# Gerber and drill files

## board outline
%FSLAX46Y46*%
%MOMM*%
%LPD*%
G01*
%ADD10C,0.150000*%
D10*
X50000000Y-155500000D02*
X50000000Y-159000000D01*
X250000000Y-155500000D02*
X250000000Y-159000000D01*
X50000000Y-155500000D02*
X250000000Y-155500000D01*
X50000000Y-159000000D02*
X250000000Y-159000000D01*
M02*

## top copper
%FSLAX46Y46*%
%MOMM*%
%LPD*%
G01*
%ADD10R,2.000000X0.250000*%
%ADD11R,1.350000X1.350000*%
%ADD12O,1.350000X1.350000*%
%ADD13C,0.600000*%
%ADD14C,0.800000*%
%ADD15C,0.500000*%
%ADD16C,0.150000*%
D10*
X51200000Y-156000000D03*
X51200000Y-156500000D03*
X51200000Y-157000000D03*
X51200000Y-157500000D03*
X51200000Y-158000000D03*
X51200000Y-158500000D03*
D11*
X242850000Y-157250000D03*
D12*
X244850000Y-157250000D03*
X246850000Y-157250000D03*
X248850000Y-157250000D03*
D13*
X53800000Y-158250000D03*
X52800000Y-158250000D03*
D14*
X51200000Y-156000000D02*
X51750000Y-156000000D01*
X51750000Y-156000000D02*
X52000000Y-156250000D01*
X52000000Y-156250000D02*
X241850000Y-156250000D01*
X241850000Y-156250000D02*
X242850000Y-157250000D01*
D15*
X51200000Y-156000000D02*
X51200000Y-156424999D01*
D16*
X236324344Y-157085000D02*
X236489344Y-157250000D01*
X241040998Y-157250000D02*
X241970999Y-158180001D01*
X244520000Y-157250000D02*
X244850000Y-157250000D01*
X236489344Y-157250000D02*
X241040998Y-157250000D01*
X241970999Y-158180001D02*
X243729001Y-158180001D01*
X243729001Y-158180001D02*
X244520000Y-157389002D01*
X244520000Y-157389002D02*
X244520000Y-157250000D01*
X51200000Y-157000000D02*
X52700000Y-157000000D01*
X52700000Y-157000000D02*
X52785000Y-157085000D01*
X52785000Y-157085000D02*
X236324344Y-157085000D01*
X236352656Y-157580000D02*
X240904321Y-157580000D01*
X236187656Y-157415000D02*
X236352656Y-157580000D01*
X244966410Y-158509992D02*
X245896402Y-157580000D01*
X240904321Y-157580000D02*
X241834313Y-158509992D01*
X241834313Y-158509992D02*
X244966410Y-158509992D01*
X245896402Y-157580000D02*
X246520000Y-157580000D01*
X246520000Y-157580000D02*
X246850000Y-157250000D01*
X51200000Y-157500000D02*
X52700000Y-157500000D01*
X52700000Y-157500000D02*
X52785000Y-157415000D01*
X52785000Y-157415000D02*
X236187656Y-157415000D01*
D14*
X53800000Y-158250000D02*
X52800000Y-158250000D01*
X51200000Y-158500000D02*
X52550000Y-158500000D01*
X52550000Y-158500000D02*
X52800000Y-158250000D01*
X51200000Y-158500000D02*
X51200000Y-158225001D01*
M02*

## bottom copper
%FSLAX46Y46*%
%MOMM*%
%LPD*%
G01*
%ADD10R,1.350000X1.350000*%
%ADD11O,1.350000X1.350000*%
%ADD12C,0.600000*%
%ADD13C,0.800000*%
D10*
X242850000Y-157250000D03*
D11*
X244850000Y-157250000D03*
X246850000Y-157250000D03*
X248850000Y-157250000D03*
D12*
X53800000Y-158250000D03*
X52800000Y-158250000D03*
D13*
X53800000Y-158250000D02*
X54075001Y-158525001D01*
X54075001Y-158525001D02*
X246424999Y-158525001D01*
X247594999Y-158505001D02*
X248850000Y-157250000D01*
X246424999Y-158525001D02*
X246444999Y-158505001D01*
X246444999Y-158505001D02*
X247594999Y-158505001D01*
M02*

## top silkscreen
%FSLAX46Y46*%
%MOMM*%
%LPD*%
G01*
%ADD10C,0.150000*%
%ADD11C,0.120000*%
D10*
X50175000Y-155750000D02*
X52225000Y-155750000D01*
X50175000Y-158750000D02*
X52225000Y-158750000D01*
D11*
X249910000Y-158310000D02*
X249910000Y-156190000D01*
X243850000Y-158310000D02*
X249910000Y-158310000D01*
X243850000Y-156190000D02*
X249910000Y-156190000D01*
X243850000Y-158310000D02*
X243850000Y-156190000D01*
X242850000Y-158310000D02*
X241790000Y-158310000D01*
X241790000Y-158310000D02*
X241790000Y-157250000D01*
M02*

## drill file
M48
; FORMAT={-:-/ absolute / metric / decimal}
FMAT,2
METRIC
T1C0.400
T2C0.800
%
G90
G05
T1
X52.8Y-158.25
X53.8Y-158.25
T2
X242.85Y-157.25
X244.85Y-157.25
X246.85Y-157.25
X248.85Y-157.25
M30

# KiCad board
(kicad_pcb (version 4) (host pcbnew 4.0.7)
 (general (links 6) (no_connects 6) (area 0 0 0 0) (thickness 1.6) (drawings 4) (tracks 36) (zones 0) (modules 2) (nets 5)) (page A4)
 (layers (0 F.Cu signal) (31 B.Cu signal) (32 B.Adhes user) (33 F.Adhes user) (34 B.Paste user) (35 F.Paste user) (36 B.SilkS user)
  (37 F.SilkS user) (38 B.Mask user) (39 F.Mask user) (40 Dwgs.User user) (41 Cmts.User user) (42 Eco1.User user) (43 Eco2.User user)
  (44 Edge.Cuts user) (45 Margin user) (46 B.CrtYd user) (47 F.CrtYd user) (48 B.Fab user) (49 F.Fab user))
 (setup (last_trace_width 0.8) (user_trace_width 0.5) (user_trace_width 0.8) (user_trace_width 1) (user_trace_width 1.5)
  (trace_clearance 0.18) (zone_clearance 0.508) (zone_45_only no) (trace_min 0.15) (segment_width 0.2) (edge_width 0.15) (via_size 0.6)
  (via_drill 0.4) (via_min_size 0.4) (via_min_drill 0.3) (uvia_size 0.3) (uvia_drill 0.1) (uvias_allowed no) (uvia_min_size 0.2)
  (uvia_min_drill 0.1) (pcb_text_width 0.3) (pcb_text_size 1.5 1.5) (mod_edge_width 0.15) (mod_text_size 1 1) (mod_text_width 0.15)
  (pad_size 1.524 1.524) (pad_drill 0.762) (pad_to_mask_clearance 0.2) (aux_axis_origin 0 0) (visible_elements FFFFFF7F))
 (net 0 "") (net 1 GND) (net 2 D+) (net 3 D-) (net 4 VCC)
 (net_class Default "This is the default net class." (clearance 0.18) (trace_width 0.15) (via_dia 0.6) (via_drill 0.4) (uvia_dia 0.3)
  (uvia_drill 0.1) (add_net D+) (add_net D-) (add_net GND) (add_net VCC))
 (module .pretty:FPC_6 (layer F.Cu) (at 51.2 157.25 270)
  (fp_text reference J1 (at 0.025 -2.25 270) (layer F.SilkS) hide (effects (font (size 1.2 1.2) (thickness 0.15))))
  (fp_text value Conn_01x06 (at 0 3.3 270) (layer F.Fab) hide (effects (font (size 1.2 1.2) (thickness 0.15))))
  (fp_line (start -1.5 1.025) (end -1.5 -1.025) (layer F.SilkS) (width 0.15))
  (fp_line (start 1.5 1.025) (end 1.5 -1.025) (layer F.SilkS) (width 0.15))
  (pad 1 smd rect (at -1.25 0 270) (size 0.25 2) (layers F.Cu F.Paste F.Mask) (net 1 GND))
  (pad 2 smd rect (at -0.75 0 270) (size 0.25 2) (layers F.Cu F.Paste F.Mask) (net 1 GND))
  (pad 3 smd rect (at -0.25 0 270) (size 0.25 2) (layers F.Cu F.Paste F.Mask) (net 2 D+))
  (pad 4 smd rect (at 0.25 0 270) (size 0.25 2) (layers F.Cu F.Paste F.Mask) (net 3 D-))
  (pad 5 smd rect (at 0.75 0 270) (size 0.25 2) (layers F.Cu F.Paste F.Mask) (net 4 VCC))
  (pad 6 smd rect (at 1.25 0 270) (size 0.25 2) (layers F.Cu F.Paste F.Mask) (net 4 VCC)))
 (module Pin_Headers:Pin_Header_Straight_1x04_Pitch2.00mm (layer F.Cu) (at 242.85 157.25 90)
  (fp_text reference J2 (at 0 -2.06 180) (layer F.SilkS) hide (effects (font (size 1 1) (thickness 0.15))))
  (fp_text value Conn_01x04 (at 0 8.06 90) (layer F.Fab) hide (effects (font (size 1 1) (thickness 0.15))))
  (fp_line (start -1.06 7.06) (end 1.06 7.06) (layer F.SilkS) (width 0.12))
  (fp_line (start -1.06 1) (end -1.06 7.06) (layer F.SilkS) (width 0.12))
  (fp_line (start 1.06 1) (end 1.06 7.06) (layer F.SilkS) (width 0.12))
  (fp_line (start -1.06 1) (end 1.06 1) (layer F.SilkS) (width 0.12))
  (fp_line (start -1.06 0) (end -1.06 -1.06) (layer F.SilkS) (width 0.12))
  (fp_line (start -1.06 -1.06) (end 0 -1.06) (layer F.SilkS) (width 0.12))
  (pad 1 thru_hole rect (at 0 0 90) (size 1.35 1.35) (drill 0.8) (layers *.Cu *.Mask) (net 1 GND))
  (pad 2 thru_hole oval (at 0 2 90) (size 1.35 1.35) (drill 0.8) (layers *.Cu *.Mask) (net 2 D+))
  (pad 3 thru_hole oval (at 0 4 90) (size 1.35 1.35) (drill 0.8) (layers *.Cu *.Mask) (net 3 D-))
  (pad 4 thru_hole oval (at 0 6 90) (size 1.35 1.35) (drill 0.8) (layers *.Cu *.Mask) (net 4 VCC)))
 (gr_line (start 50 155.5) (end 50 159) (layer Edge.Cuts) (width 0.15))
 (gr_line (start 250 155.5) (end 250 159) (layer Edge.Cuts) (width 0.15))
 (gr_line (start 50 155.5) (end 250 155.5) (layer Edge.Cuts) (width 0.15))
 (gr_line (start 50 159) (end 250 159) (layer Edge.Cuts) (width 0.15))
 (segment (start 51.2 156) (end 51.75 156) (width 0.8) (layer F.Cu) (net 1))
 (segment (start 51.75 156) (end 52 156.25) (width 0.8) (layer F.Cu) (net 1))
 (segment (start 52 156.25) (end 241.85 156.25) (width 0.8) (layer F.Cu) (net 1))
 (segment (start 241.85 156.25) (end 242.85 157.25) (width 0.8) (layer F.Cu) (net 1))
 (segment (start 51.2 156) (end 51.2 156.424999) (width 0.5) (layer F.Cu) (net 1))
 (segment (start 236.324344 157.085) (end 236.489344 157.25) (width 0.15) (layer F.Cu) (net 2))
 (segment (start 241.040998 157.25) (end 241.970999 158.180001) (width 0.15) (layer F.Cu) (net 2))
 (segment (start 244.52 157.25) (end 244.85 157.25) (width 0.15) (layer F.Cu) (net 2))
 (segment (start 236.489344 157.25) (end 241.040998 157.25) (width 0.15) (layer F.Cu) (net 2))
 (segment (start 241.970999 158.180001) (end 243.729001 158.180001) (width 0.15) (layer F.Cu) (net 2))
 (segment (start 243.729001 158.180001) (end 244.52 157.389002) (width 0.15) (layer F.Cu) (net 2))
 (segment (start 244.52 157.389002) (end 244.52 157.25) (width 0.15) (layer F.Cu) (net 2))
 (segment (start 51.2 157) (end 52.7 157) (width 0.15) (layer F.Cu) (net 2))
 (segment (start 52.7 157) (end 52.785 157.085) (width 0.15) (layer F.Cu) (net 2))
 (segment (start 52.785 157.085) (end 236.324344 157.085) (width 0.15) (layer F.Cu) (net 2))
 (segment (start 236.352656 157.58) (end 240.904321 157.58) (width 0.15) (layer F.Cu) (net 3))
 (segment (start 236.187656 157.415) (end 236.352656 157.58) (width 0.15) (layer F.Cu) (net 3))
 (segment (start 244.96641 158.509992) (end 245.896402 157.58) (width 0.15) (layer F.Cu) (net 3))
 (segment (start 240.904321 157.58) (end 241.834313 158.509992) (width 0.15) (layer F.Cu) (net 3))
 (segment (start 241.834313 158.509992) (end 244.96641 158.509992) (width 0.15) (layer F.Cu) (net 3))
 (segment (start 245.896402 157.58) (end 246.52 157.58) (width 0.15) (layer F.Cu) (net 3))
 (segment (start 246.52 157.58) (end 246.85 157.25) (width 0.15) (layer F.Cu) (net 3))
 (segment (start 51.2 157.5) (end 52.7 157.5) (width 0.15) (layer F.Cu) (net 3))
 (segment (start 52.7 157.5) (end 52.785 157.415) (width 0.15) (layer F.Cu) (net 3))
 (segment (start 52.785 157.415) (end 236.187656 157.415) (width 0.15) (layer F.Cu) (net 3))
 (segment (start 53.8 158.25) (end 54.075001 158.525001) (width 0.8) (layer B.Cu) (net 4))
 (segment (start 54.075001 158.525001) (end 246.424999 158.525001) (width 0.8) (layer B.Cu) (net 4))
 (segment (start 247.594999 158.505001) (end 248.85 157.25) (width 0.8) (layer B.Cu) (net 4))
 (segment (start 246.424999 158.525001) (end 246.444999 158.505001) (width 0.8) (layer B.Cu) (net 4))
 (segment (start 246.444999 158.505001) (end 247.594999 158.505001) (width 0.8) (layer B.Cu) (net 4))
 (segment (start 53.8 158.25) (end 52.8 158.25) (width 0.8) (layer F.Cu) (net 4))
 (via (at 53.8 158.25) (size 0.6) (drill 0.4) (layers F.Cu B.Cu) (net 4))
 (segment (start 51.2 158.5) (end 52.55 158.5) (width 0.8) (layer F.Cu) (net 4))
 (segment (start 52.55 158.5) (end 52.8 158.25) (width 0.8) (layer F.Cu) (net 4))
 (via (at 52.8 158.25) (size 0.6) (drill 0.4) (layers F.Cu B.Cu) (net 4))
 (segment (start 51.2 158.5) (end 51.2 158.225001) (width 0.8) (layer F.Cu) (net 4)))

